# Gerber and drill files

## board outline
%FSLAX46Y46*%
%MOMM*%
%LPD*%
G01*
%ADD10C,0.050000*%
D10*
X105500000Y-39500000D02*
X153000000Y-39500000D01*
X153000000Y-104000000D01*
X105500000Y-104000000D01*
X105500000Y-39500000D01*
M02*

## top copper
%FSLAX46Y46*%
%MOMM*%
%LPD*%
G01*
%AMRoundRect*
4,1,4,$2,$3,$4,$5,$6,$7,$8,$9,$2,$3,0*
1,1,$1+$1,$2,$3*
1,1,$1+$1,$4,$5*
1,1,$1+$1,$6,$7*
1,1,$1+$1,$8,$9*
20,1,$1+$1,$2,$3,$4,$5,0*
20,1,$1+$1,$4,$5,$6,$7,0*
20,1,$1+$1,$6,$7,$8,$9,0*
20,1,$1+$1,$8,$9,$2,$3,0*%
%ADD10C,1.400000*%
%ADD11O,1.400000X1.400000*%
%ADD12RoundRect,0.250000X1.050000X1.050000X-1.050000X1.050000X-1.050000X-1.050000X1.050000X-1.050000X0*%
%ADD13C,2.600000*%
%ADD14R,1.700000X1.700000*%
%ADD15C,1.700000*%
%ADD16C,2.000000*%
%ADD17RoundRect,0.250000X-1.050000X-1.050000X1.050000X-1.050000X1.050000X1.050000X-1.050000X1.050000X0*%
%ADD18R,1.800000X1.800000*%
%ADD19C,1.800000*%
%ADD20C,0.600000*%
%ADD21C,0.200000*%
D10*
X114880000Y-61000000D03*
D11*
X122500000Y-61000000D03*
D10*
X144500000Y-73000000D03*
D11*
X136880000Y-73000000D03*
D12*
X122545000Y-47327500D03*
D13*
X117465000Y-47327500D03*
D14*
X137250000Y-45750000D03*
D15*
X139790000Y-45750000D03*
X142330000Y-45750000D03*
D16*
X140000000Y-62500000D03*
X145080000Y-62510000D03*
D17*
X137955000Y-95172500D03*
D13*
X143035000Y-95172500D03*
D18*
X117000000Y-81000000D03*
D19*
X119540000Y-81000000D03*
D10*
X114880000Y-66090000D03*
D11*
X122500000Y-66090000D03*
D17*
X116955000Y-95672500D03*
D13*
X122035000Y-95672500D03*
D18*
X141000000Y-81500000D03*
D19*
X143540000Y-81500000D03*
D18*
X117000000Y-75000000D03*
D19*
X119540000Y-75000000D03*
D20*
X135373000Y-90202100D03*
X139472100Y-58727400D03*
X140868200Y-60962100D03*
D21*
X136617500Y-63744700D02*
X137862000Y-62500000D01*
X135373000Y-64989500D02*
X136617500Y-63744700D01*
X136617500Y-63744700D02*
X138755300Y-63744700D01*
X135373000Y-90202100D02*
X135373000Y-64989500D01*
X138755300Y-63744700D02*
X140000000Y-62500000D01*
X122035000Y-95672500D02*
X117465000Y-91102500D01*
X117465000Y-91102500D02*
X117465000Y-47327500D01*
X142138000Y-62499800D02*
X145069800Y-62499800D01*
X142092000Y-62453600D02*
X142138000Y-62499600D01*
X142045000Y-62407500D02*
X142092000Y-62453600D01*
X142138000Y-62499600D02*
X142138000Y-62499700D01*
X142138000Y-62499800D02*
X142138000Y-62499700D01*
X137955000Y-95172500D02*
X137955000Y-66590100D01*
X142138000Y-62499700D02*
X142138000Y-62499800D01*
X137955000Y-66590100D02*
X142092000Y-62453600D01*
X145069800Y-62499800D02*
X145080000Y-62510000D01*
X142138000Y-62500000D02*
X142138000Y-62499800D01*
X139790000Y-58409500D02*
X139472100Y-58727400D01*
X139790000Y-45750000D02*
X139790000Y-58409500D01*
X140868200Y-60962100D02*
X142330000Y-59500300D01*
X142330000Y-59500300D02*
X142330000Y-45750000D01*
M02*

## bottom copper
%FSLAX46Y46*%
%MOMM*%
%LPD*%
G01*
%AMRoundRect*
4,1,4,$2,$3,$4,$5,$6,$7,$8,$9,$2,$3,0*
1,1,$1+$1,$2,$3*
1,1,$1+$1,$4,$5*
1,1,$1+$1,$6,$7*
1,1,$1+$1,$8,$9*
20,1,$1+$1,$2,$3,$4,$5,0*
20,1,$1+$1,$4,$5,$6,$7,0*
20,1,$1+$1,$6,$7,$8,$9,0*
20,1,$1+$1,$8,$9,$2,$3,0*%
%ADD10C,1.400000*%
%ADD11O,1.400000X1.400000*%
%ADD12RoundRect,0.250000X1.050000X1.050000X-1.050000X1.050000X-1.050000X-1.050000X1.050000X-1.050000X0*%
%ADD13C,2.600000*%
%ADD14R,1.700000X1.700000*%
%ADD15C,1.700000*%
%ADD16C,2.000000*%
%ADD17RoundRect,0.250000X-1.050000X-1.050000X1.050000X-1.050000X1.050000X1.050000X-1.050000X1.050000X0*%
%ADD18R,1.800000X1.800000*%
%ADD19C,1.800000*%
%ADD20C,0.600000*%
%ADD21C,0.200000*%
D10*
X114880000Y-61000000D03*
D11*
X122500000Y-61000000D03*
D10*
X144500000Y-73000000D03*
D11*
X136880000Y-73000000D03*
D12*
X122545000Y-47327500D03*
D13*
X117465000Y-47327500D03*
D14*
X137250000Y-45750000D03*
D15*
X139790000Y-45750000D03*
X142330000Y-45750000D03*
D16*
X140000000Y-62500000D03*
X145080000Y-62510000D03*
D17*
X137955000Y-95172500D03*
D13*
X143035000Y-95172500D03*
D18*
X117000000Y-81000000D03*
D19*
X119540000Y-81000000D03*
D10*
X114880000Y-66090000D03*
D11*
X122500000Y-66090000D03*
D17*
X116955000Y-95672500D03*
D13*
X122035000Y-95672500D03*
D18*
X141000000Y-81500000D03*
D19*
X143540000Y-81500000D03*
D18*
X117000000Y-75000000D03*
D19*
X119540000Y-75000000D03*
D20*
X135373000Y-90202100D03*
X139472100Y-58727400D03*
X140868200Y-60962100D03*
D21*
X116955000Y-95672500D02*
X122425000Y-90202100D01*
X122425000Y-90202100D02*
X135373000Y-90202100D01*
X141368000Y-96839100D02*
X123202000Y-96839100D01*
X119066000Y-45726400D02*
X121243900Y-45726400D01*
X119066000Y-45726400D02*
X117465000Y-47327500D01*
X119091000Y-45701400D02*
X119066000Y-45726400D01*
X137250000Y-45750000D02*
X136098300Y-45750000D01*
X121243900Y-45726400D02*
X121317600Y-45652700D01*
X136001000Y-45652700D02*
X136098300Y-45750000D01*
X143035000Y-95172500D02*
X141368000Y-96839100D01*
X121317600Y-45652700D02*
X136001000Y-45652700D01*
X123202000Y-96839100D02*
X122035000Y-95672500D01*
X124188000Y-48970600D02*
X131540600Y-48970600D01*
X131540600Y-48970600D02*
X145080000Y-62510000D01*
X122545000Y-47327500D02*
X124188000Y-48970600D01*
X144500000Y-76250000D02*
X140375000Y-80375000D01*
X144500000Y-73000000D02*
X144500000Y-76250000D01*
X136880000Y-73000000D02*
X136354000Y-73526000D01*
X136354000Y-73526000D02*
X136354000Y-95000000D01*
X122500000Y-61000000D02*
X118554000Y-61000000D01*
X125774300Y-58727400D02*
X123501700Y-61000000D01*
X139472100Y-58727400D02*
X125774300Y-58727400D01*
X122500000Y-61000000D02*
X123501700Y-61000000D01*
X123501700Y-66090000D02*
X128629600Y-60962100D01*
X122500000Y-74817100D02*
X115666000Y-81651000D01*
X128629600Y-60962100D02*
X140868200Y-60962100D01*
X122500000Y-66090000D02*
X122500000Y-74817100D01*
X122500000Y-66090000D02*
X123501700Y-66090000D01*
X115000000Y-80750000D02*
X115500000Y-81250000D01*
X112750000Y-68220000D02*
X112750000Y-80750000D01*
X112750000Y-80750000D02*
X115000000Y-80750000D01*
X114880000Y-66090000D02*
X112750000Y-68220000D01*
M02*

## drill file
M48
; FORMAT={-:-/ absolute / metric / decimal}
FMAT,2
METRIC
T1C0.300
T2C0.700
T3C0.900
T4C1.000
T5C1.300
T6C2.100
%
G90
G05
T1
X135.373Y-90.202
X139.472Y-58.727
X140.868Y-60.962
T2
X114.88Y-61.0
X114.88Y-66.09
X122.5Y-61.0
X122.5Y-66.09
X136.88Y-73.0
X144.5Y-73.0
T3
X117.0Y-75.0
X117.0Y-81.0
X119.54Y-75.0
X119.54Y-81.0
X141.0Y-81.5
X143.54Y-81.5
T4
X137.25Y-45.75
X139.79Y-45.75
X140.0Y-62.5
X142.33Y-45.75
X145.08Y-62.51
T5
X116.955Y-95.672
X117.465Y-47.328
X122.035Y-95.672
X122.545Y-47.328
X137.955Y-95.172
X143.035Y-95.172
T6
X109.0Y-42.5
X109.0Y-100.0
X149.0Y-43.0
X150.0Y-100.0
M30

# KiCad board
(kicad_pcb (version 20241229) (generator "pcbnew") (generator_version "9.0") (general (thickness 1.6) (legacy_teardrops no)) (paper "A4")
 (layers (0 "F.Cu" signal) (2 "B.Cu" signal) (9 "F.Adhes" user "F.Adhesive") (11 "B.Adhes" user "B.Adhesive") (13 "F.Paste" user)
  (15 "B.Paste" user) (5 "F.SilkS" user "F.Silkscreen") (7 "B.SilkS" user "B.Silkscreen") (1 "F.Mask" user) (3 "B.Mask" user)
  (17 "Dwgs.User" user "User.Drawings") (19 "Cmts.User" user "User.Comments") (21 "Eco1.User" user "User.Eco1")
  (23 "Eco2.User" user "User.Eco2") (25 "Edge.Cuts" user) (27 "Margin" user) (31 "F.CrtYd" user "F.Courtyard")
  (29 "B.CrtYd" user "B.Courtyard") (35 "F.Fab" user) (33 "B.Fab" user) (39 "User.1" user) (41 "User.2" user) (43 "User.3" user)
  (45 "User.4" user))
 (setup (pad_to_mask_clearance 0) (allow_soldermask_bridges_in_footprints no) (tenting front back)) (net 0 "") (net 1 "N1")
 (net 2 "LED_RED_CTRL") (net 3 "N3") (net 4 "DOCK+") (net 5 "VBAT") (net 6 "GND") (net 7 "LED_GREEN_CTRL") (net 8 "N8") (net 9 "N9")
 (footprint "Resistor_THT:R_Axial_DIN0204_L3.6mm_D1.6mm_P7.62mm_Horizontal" (layer "F.Cu") (at 114.88 61)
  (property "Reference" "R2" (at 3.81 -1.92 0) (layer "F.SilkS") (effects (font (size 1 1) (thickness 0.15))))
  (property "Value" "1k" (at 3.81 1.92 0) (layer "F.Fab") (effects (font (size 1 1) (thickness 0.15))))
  (pad "1" thru_hole circle (at 0 0) (size 1.4 1.4) (drill 0.7) (layers "*.Cu" "*.Mask") (remove_unused_layers no) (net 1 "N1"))
  (pad "2" thru_hole oval (at 7.62 0) (size 1.4 1.4) (drill 0.7) (layers "*.Cu" "*.Mask") (remove_unused_layers no) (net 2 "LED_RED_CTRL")))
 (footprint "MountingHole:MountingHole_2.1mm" (layer "F.Cu") (at 109 100)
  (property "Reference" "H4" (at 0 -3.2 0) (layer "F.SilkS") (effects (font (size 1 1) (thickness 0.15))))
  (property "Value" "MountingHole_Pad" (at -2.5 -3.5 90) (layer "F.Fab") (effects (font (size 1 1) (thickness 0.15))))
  (pad "" np_thru_hole circle (at 0 0) (size 2.1 2.1) (drill 2.1) (layers "*.Cu" "*.Mask")))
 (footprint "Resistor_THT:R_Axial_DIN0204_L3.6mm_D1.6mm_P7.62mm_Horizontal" (layer "F.Cu") (at 144.5 73 180)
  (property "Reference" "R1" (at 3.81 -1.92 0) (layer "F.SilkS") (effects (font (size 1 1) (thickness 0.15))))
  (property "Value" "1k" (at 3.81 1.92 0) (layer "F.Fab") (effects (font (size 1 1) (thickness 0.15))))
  (pad "1" thru_hole circle (at 0 0 180) (size 1.4 1.4) (drill 0.7) (layers "*.Cu" "*.Mask") (remove_unused_layers no) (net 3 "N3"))
  (pad "2" thru_hole oval (at 7.62 0 180) (size 1.4 1.4) (drill 0.7) (layers "*.Cu" "*.Mask") (remove_unused_layers no) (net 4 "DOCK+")))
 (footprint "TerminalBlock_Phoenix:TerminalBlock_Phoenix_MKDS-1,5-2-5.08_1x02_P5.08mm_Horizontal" (layer "F.Cu") (at 122.545 47.3275 180)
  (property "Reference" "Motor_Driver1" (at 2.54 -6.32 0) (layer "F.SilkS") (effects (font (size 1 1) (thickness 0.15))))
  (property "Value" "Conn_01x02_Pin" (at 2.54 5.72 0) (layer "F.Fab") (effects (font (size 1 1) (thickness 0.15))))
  (pad "1" thru_hole roundrect (at 0 0 180) (size 2.6 2.6) (drill 1.3) (layers "*.Cu" "*.Mask") (remove_unused_layers no)
   (roundrect_rratio 0.096154) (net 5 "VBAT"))
  (pad "2" thru_hole circle (at 5.08 0 180) (size 2.6 2.6) (drill 1.3) (layers "*.Cu" "*.Mask") (remove_unused_layers no) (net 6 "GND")))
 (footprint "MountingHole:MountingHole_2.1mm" (layer "F.Cu") (at 150 100)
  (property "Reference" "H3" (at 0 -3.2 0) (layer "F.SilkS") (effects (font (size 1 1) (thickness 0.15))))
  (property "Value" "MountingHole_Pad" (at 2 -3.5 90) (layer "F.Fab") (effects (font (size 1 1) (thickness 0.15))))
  (pad "" np_thru_hole circle (at 0 0) (size 2.1 2.1) (drill 2.1) (layers "*.Cu" "*.Mask")))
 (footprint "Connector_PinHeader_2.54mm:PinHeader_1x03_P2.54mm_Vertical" (layer "F.Cu") (at 137.25 45.75 90)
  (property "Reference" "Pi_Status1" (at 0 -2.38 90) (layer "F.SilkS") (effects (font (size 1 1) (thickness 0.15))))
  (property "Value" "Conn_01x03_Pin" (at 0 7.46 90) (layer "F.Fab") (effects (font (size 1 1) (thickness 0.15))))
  (pad "1" thru_hole rect (at 0 0 90) (size 1.7 1.7) (drill 1) (layers "*.Cu" "*.Mask") (remove_unused_layers no) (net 6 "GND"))
  (pad "2" thru_hole circle (at 0 2.54 90) (size 1.7 1.7) (drill 1) (layers "*.Cu" "*.Mask") (remove_unused_layers no)
   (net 2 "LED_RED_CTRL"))
  (pad "3" thru_hole circle (at 0 5.08 90) (size 1.7 1.7) (drill 1) (layers "*.Cu" "*.Mask") (remove_unused_layers no)
   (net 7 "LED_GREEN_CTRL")))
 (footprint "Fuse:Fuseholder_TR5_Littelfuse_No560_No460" (layer "F.Cu") (at 140 62.5)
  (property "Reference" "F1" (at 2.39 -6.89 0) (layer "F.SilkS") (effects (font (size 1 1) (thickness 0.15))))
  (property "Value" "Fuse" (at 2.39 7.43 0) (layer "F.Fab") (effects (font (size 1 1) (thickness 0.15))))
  (pad "1" thru_hole circle (at 0 0) (size 2 2) (drill 1) (layers "*.Cu" "*.Mask") (remove_unused_layers no) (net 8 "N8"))
  (pad "2" thru_hole circle (at 5.08 0.01) (size 2 2) (drill 1) (layers "*.Cu" "*.Mask") (remove_unused_layers no) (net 5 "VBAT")))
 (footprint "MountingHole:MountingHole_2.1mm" (layer "F.Cu") (at 149 43)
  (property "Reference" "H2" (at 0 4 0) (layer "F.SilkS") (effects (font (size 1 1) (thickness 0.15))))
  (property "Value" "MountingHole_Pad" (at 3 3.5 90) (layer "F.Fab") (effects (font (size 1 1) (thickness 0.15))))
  (pad "" np_thru_hole circle (at 0 0) (size 2.1 2.1) (drill 2.1) (layers "*.Cu" "*.Mask")))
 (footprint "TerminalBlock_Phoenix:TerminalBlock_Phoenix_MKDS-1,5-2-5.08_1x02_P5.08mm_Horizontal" (layer "F.Cu") (at 137.955 95.1725)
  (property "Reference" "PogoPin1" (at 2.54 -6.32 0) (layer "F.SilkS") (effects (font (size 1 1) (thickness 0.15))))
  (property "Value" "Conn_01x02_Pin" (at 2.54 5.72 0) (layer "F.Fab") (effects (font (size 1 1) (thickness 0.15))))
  (pad "1" thru_hole roundrect (at 0 0) (size 2.6 2.6) (drill 1.3) (layers "*.Cu" "*.Mask") (remove_unused_layers no)
   (roundrect_rratio 0.096154) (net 5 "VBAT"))
  (pad "2" thru_hole circle (at 5.08 0) (size 2.6 2.6) (drill 1.3) (layers "*.Cu" "*.Mask") (remove_unused_layers no) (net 6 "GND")))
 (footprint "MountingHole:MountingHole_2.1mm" (layer "F.Cu") (at 109 42.5)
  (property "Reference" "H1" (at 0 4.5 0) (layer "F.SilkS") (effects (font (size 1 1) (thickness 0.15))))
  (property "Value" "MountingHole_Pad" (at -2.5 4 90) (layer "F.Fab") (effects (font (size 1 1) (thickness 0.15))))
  (pad "" np_thru_hole circle (at 0 0) (size 2.1 2.1) (drill 2.1) (layers "*.Cu" "*.Mask")))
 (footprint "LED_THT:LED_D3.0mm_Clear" (layer "F.Cu") (at 117 81)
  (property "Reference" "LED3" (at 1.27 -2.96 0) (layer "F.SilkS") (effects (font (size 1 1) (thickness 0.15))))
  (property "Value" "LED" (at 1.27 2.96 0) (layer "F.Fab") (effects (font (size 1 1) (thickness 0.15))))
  (pad "1" thru_hole rect (at 0 0) (size 1.8 1.8) (drill 0.9) (layers "*.Cu" "*.Mask") (remove_unused_layers no))
  (pad "2" thru_hole circle (at 2.54 0) (size 1.8 1.8) (drill 0.9) (layers "*.Cu" "*.Mask") (remove_unused_layers no)))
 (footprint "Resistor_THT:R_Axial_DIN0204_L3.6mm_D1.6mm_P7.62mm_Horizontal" (layer "F.Cu") (at 114.88 66.09)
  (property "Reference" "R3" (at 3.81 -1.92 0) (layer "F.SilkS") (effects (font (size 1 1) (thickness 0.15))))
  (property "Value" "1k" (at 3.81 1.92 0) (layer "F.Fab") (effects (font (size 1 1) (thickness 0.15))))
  (pad "1" thru_hole circle (at 0 0) (size 1.4 1.4) (drill 0.7) (layers "*.Cu" "*.Mask") (remove_unused_layers no) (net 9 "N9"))
  (pad "2" thru_hole oval (at 7.62 0) (size 1.4 1.4) (drill 0.7) (layers "*.Cu" "*.Mask") (remove_unused_layers no) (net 7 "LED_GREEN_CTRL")))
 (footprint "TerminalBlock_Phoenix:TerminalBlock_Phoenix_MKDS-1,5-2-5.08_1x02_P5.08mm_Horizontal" (layer "F.Cu") (at 116.955 95.6725)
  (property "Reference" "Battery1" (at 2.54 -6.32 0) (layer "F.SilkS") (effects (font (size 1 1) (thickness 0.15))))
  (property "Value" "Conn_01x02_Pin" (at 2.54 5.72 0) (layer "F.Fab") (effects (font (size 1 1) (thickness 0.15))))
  (pad "1" thru_hole roundrect (at 0 0) (size 2.6 2.6) (drill 1.3) (layers "*.Cu" "*.Mask") (remove_unused_layers no)
   (roundrect_rratio 0.096154) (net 8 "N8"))
  (pad "2" thru_hole circle (at 5.08 0) (size 2.6 2.6) (drill 1.3) (layers "*.Cu" "*.Mask") (remove_unused_layers no) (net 6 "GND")))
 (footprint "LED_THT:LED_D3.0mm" (layer "F.Cu") (at 141 81.5)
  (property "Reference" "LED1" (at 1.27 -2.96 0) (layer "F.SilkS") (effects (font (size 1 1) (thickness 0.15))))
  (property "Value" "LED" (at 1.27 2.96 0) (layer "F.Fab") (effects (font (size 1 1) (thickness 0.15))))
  (pad "1" thru_hole rect (at 0 0) (size 1.8 1.8) (drill 0.9) (layers "*.Cu" "*.Mask") (remove_unused_layers no))
  (pad "2" thru_hole circle (at 2.54 0) (size 1.8 1.8) (drill 0.9) (layers "*.Cu" "*.Mask") (remove_unused_layers no)))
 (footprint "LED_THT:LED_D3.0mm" (layer "F.Cu") (at 117 75)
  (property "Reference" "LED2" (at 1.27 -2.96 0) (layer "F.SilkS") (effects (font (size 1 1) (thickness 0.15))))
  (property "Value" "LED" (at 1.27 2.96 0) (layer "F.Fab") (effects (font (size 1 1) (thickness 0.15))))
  (pad "1" thru_hole rect (at 0 0) (size 1.8 1.8) (drill 0.9) (layers "*.Cu" "*.Mask") (remove_unused_layers no))
  (pad "2" thru_hole circle (at 2.54 0) (size 1.8 1.8) (drill 0.9) (layers "*.Cu" "*.Mask") (remove_unused_layers no)))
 (gr_rect (start 105.5 39.5) (end 153 104) (stroke (width 0.05) (type default)) (fill no) (layer "Edge.Cuts"))
 (segment (start 136.6175 63.7447) (end 137.862 62.5) (width 0.2) (layer "F.Cu") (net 8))
 (segment (start 135.373 64.9895) (end 136.6175 63.7447) (width 0.2) (layer "F.Cu") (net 8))
 (segment (start 136.6175 63.7447) (end 138.7553 63.7447) (width 0.2) (layer "F.Cu") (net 8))
 (segment (start 135.373 90.2021) (end 135.373 64.9895) (width 0.2) (layer "F.Cu") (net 8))
 (segment (start 138.7553 63.7447) (end 140 62.5) (width 0.2) (layer "F.Cu") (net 8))
 (via (at 135.373 90.2021) (size 0.6) (drill 0.3) (layers "F.Cu" "B.Cu") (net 8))
 (segment (start 116.955 95.6725) (end 122.425 90.2021) (width 0.2) (layer "B.Cu") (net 8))
 (segment (start 122.425 90.2021) (end 135.373 90.2021) (width 0.2) (layer "B.Cu") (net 8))
 (segment (start 122.035 95.6725) (end 117.465 91.1025) (width 0.2) (layer "F.Cu") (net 6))
 (segment (start 117.465 91.1025) (end 117.465 47.3275) (width 0.2) (layer "F.Cu") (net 6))
 (segment (start 141.368 96.8391) (end 123.202 96.8391) (width 0.2) (layer "B.Cu") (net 6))
 (segment (start 119.066 45.7264) (end 121.2439 45.7264) (width 0.2) (layer "B.Cu") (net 6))
 (segment (start 119.066 45.7264) (end 117.465 47.3275) (width 0.2) (layer "B.Cu") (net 6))
 (segment (start 119.091 45.7014) (end 119.066 45.7264) (width 0.2) (layer "B.Cu") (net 6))
 (segment (start 137.25 45.75) (end 136.0983 45.75) (width 0.2) (layer "B.Cu") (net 6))
 (segment (start 121.2439 45.7264) (end 121.3176 45.6527) (width 0.2) (layer "B.Cu") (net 6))
 (segment (start 136.001 45.6527) (end 136.0983 45.75) (width 0.2) (layer "B.Cu") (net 6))
 (segment (start 143.035 95.1725) (end 141.368 96.8391) (width 0.2) (layer "B.Cu") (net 6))
 (segment (start 121.3176 45.6527) (end 136.001 45.6527) (width 0.2) (layer "B.Cu") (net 6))
 (segment (start 123.202 96.8391) (end 122.035 95.6725) (width 0.2) (layer "B.Cu") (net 6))
 (segment (start 142.138 62.4998) (end 145.0698 62.4998) (width 0.2) (layer "F.Cu") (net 5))
 (segment (start 142.092 62.4536) (end 142.138 62.4996) (width 0.2) (layer "F.Cu") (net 5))
 (segment (start 142.045 62.4075) (end 142.092 62.4536) (width 0.2) (layer "F.Cu") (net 5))
 (segment (start 142.138 62.4996) (end 142.138 62.4997) (width 0.2) (layer "F.Cu") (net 5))
 (segment (start 142.138 62.4998) (end 142.138 62.4997) (width 0.2) (layer "F.Cu") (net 5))
 (segment (start 137.955 95.1725) (end 137.955 66.5901) (width 0.2) (layer "F.Cu") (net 5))
 (segment (start 142.138 62.4997) (end 142.138 62.4998) (width 0.2) (layer "F.Cu") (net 5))
 (segment (start 137.955 66.5901) (end 142.092 62.4536) (width 0.2) (layer "F.Cu") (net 5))
 (segment (start 145.0698 62.4998) (end 145.08 62.51) (width 0.2) (layer "F.Cu") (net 5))
 (segment (start 142.138 62.5) (end 142.138 62.4998) (width 0.2) (layer "F.Cu") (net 5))
 (segment (start 124.188 48.9706) (end 131.5406 48.9706) (width 0.2) (layer "B.Cu") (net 5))
 (segment (start 131.5406 48.9706) (end 145.08 62.51) (width 0.2) (layer "B.Cu") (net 5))
 (segment (start 122.545 47.3275) (end 124.188 48.9706) (width 0.2) (layer "B.Cu") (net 5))
 (segment (start 144.5 76.25) (end 140.375 80.375) (width 0.2) (layer "B.Cu") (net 3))
 (segment (start 144.5 73) (end 144.5 76.25) (width 0.2) (layer "B.Cu") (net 3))
 (segment (start 136.88 73) (end 136.354 73.526) (width 0.2) (layer "B.Cu") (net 4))
 (segment (start 136.354 73.526) (end 136.354 95) (width 0.2) (layer "B.Cu") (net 4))
 (segment (start 139.79 58.4095) (end 139.4721 58.7274) (width 0.2) (layer "F.Cu") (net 2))
 (segment (start 139.79 45.75) (end 139.79 58.4095) (width 0.2) (layer "F.Cu") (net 2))
 (via (at 139.4721 58.7274) (size 0.6) (drill 0.3) (layers "F.Cu" "B.Cu") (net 2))
 (segment (start 122.5 61) (end 118.554 61) (width 0.2) (layer "B.Cu") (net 2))
 (segment (start 125.7743 58.7274) (end 123.5017 61) (width 0.2) (layer "B.Cu") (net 2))
 (segment (start 139.4721 58.7274) (end 125.7743 58.7274) (width 0.2) (layer "B.Cu") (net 2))
 (segment (start 122.5 61) (end 123.5017 61) (width 0.2) (layer "B.Cu") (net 2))
 (segment (start 140.8682 60.9621) (end 142.33 59.5003) (width 0.2) (layer "F.Cu") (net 7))
 (segment (start 142.33 59.5003) (end 142.33 45.75) (width 0.2) (layer "F.Cu") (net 7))
 (via (at 140.8682 60.9621) (size 0.6) (drill 0.3) (layers "F.Cu" "B.Cu") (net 7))
 (segment (start 123.5017 66.09) (end 128.6296 60.9621) (width 0.2) (layer "B.Cu") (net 7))
 (segment (start 122.5 74.8171) (end 115.666 81.651) (width 0.2) (layer "B.Cu") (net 7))
 (segment (start 128.6296 60.9621) (end 140.8682 60.9621) (width 0.2) (layer "B.Cu") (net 7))
 (segment (start 122.5 66.09) (end 122.5 74.8171) (width 0.2) (layer "B.Cu") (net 7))
 (segment (start 122.5 66.09) (end 123.5017 66.09) (width 0.2) (layer "B.Cu") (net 7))
 (segment (start 115 80.75) (end 115.5 81.25) (width 0.2) (layer "B.Cu") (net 9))
 (segment (start 112.75 68.22) (end 112.75 80.75) (width 0.2) (layer "B.Cu") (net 9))
 (segment (start 112.75 80.75) (end 115 80.75) (width 0.2) (layer "B.Cu") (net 9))
 (segment (start 114.88 66.09) (end 112.75 68.22) (width 0.2) (layer "B.Cu") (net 9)))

